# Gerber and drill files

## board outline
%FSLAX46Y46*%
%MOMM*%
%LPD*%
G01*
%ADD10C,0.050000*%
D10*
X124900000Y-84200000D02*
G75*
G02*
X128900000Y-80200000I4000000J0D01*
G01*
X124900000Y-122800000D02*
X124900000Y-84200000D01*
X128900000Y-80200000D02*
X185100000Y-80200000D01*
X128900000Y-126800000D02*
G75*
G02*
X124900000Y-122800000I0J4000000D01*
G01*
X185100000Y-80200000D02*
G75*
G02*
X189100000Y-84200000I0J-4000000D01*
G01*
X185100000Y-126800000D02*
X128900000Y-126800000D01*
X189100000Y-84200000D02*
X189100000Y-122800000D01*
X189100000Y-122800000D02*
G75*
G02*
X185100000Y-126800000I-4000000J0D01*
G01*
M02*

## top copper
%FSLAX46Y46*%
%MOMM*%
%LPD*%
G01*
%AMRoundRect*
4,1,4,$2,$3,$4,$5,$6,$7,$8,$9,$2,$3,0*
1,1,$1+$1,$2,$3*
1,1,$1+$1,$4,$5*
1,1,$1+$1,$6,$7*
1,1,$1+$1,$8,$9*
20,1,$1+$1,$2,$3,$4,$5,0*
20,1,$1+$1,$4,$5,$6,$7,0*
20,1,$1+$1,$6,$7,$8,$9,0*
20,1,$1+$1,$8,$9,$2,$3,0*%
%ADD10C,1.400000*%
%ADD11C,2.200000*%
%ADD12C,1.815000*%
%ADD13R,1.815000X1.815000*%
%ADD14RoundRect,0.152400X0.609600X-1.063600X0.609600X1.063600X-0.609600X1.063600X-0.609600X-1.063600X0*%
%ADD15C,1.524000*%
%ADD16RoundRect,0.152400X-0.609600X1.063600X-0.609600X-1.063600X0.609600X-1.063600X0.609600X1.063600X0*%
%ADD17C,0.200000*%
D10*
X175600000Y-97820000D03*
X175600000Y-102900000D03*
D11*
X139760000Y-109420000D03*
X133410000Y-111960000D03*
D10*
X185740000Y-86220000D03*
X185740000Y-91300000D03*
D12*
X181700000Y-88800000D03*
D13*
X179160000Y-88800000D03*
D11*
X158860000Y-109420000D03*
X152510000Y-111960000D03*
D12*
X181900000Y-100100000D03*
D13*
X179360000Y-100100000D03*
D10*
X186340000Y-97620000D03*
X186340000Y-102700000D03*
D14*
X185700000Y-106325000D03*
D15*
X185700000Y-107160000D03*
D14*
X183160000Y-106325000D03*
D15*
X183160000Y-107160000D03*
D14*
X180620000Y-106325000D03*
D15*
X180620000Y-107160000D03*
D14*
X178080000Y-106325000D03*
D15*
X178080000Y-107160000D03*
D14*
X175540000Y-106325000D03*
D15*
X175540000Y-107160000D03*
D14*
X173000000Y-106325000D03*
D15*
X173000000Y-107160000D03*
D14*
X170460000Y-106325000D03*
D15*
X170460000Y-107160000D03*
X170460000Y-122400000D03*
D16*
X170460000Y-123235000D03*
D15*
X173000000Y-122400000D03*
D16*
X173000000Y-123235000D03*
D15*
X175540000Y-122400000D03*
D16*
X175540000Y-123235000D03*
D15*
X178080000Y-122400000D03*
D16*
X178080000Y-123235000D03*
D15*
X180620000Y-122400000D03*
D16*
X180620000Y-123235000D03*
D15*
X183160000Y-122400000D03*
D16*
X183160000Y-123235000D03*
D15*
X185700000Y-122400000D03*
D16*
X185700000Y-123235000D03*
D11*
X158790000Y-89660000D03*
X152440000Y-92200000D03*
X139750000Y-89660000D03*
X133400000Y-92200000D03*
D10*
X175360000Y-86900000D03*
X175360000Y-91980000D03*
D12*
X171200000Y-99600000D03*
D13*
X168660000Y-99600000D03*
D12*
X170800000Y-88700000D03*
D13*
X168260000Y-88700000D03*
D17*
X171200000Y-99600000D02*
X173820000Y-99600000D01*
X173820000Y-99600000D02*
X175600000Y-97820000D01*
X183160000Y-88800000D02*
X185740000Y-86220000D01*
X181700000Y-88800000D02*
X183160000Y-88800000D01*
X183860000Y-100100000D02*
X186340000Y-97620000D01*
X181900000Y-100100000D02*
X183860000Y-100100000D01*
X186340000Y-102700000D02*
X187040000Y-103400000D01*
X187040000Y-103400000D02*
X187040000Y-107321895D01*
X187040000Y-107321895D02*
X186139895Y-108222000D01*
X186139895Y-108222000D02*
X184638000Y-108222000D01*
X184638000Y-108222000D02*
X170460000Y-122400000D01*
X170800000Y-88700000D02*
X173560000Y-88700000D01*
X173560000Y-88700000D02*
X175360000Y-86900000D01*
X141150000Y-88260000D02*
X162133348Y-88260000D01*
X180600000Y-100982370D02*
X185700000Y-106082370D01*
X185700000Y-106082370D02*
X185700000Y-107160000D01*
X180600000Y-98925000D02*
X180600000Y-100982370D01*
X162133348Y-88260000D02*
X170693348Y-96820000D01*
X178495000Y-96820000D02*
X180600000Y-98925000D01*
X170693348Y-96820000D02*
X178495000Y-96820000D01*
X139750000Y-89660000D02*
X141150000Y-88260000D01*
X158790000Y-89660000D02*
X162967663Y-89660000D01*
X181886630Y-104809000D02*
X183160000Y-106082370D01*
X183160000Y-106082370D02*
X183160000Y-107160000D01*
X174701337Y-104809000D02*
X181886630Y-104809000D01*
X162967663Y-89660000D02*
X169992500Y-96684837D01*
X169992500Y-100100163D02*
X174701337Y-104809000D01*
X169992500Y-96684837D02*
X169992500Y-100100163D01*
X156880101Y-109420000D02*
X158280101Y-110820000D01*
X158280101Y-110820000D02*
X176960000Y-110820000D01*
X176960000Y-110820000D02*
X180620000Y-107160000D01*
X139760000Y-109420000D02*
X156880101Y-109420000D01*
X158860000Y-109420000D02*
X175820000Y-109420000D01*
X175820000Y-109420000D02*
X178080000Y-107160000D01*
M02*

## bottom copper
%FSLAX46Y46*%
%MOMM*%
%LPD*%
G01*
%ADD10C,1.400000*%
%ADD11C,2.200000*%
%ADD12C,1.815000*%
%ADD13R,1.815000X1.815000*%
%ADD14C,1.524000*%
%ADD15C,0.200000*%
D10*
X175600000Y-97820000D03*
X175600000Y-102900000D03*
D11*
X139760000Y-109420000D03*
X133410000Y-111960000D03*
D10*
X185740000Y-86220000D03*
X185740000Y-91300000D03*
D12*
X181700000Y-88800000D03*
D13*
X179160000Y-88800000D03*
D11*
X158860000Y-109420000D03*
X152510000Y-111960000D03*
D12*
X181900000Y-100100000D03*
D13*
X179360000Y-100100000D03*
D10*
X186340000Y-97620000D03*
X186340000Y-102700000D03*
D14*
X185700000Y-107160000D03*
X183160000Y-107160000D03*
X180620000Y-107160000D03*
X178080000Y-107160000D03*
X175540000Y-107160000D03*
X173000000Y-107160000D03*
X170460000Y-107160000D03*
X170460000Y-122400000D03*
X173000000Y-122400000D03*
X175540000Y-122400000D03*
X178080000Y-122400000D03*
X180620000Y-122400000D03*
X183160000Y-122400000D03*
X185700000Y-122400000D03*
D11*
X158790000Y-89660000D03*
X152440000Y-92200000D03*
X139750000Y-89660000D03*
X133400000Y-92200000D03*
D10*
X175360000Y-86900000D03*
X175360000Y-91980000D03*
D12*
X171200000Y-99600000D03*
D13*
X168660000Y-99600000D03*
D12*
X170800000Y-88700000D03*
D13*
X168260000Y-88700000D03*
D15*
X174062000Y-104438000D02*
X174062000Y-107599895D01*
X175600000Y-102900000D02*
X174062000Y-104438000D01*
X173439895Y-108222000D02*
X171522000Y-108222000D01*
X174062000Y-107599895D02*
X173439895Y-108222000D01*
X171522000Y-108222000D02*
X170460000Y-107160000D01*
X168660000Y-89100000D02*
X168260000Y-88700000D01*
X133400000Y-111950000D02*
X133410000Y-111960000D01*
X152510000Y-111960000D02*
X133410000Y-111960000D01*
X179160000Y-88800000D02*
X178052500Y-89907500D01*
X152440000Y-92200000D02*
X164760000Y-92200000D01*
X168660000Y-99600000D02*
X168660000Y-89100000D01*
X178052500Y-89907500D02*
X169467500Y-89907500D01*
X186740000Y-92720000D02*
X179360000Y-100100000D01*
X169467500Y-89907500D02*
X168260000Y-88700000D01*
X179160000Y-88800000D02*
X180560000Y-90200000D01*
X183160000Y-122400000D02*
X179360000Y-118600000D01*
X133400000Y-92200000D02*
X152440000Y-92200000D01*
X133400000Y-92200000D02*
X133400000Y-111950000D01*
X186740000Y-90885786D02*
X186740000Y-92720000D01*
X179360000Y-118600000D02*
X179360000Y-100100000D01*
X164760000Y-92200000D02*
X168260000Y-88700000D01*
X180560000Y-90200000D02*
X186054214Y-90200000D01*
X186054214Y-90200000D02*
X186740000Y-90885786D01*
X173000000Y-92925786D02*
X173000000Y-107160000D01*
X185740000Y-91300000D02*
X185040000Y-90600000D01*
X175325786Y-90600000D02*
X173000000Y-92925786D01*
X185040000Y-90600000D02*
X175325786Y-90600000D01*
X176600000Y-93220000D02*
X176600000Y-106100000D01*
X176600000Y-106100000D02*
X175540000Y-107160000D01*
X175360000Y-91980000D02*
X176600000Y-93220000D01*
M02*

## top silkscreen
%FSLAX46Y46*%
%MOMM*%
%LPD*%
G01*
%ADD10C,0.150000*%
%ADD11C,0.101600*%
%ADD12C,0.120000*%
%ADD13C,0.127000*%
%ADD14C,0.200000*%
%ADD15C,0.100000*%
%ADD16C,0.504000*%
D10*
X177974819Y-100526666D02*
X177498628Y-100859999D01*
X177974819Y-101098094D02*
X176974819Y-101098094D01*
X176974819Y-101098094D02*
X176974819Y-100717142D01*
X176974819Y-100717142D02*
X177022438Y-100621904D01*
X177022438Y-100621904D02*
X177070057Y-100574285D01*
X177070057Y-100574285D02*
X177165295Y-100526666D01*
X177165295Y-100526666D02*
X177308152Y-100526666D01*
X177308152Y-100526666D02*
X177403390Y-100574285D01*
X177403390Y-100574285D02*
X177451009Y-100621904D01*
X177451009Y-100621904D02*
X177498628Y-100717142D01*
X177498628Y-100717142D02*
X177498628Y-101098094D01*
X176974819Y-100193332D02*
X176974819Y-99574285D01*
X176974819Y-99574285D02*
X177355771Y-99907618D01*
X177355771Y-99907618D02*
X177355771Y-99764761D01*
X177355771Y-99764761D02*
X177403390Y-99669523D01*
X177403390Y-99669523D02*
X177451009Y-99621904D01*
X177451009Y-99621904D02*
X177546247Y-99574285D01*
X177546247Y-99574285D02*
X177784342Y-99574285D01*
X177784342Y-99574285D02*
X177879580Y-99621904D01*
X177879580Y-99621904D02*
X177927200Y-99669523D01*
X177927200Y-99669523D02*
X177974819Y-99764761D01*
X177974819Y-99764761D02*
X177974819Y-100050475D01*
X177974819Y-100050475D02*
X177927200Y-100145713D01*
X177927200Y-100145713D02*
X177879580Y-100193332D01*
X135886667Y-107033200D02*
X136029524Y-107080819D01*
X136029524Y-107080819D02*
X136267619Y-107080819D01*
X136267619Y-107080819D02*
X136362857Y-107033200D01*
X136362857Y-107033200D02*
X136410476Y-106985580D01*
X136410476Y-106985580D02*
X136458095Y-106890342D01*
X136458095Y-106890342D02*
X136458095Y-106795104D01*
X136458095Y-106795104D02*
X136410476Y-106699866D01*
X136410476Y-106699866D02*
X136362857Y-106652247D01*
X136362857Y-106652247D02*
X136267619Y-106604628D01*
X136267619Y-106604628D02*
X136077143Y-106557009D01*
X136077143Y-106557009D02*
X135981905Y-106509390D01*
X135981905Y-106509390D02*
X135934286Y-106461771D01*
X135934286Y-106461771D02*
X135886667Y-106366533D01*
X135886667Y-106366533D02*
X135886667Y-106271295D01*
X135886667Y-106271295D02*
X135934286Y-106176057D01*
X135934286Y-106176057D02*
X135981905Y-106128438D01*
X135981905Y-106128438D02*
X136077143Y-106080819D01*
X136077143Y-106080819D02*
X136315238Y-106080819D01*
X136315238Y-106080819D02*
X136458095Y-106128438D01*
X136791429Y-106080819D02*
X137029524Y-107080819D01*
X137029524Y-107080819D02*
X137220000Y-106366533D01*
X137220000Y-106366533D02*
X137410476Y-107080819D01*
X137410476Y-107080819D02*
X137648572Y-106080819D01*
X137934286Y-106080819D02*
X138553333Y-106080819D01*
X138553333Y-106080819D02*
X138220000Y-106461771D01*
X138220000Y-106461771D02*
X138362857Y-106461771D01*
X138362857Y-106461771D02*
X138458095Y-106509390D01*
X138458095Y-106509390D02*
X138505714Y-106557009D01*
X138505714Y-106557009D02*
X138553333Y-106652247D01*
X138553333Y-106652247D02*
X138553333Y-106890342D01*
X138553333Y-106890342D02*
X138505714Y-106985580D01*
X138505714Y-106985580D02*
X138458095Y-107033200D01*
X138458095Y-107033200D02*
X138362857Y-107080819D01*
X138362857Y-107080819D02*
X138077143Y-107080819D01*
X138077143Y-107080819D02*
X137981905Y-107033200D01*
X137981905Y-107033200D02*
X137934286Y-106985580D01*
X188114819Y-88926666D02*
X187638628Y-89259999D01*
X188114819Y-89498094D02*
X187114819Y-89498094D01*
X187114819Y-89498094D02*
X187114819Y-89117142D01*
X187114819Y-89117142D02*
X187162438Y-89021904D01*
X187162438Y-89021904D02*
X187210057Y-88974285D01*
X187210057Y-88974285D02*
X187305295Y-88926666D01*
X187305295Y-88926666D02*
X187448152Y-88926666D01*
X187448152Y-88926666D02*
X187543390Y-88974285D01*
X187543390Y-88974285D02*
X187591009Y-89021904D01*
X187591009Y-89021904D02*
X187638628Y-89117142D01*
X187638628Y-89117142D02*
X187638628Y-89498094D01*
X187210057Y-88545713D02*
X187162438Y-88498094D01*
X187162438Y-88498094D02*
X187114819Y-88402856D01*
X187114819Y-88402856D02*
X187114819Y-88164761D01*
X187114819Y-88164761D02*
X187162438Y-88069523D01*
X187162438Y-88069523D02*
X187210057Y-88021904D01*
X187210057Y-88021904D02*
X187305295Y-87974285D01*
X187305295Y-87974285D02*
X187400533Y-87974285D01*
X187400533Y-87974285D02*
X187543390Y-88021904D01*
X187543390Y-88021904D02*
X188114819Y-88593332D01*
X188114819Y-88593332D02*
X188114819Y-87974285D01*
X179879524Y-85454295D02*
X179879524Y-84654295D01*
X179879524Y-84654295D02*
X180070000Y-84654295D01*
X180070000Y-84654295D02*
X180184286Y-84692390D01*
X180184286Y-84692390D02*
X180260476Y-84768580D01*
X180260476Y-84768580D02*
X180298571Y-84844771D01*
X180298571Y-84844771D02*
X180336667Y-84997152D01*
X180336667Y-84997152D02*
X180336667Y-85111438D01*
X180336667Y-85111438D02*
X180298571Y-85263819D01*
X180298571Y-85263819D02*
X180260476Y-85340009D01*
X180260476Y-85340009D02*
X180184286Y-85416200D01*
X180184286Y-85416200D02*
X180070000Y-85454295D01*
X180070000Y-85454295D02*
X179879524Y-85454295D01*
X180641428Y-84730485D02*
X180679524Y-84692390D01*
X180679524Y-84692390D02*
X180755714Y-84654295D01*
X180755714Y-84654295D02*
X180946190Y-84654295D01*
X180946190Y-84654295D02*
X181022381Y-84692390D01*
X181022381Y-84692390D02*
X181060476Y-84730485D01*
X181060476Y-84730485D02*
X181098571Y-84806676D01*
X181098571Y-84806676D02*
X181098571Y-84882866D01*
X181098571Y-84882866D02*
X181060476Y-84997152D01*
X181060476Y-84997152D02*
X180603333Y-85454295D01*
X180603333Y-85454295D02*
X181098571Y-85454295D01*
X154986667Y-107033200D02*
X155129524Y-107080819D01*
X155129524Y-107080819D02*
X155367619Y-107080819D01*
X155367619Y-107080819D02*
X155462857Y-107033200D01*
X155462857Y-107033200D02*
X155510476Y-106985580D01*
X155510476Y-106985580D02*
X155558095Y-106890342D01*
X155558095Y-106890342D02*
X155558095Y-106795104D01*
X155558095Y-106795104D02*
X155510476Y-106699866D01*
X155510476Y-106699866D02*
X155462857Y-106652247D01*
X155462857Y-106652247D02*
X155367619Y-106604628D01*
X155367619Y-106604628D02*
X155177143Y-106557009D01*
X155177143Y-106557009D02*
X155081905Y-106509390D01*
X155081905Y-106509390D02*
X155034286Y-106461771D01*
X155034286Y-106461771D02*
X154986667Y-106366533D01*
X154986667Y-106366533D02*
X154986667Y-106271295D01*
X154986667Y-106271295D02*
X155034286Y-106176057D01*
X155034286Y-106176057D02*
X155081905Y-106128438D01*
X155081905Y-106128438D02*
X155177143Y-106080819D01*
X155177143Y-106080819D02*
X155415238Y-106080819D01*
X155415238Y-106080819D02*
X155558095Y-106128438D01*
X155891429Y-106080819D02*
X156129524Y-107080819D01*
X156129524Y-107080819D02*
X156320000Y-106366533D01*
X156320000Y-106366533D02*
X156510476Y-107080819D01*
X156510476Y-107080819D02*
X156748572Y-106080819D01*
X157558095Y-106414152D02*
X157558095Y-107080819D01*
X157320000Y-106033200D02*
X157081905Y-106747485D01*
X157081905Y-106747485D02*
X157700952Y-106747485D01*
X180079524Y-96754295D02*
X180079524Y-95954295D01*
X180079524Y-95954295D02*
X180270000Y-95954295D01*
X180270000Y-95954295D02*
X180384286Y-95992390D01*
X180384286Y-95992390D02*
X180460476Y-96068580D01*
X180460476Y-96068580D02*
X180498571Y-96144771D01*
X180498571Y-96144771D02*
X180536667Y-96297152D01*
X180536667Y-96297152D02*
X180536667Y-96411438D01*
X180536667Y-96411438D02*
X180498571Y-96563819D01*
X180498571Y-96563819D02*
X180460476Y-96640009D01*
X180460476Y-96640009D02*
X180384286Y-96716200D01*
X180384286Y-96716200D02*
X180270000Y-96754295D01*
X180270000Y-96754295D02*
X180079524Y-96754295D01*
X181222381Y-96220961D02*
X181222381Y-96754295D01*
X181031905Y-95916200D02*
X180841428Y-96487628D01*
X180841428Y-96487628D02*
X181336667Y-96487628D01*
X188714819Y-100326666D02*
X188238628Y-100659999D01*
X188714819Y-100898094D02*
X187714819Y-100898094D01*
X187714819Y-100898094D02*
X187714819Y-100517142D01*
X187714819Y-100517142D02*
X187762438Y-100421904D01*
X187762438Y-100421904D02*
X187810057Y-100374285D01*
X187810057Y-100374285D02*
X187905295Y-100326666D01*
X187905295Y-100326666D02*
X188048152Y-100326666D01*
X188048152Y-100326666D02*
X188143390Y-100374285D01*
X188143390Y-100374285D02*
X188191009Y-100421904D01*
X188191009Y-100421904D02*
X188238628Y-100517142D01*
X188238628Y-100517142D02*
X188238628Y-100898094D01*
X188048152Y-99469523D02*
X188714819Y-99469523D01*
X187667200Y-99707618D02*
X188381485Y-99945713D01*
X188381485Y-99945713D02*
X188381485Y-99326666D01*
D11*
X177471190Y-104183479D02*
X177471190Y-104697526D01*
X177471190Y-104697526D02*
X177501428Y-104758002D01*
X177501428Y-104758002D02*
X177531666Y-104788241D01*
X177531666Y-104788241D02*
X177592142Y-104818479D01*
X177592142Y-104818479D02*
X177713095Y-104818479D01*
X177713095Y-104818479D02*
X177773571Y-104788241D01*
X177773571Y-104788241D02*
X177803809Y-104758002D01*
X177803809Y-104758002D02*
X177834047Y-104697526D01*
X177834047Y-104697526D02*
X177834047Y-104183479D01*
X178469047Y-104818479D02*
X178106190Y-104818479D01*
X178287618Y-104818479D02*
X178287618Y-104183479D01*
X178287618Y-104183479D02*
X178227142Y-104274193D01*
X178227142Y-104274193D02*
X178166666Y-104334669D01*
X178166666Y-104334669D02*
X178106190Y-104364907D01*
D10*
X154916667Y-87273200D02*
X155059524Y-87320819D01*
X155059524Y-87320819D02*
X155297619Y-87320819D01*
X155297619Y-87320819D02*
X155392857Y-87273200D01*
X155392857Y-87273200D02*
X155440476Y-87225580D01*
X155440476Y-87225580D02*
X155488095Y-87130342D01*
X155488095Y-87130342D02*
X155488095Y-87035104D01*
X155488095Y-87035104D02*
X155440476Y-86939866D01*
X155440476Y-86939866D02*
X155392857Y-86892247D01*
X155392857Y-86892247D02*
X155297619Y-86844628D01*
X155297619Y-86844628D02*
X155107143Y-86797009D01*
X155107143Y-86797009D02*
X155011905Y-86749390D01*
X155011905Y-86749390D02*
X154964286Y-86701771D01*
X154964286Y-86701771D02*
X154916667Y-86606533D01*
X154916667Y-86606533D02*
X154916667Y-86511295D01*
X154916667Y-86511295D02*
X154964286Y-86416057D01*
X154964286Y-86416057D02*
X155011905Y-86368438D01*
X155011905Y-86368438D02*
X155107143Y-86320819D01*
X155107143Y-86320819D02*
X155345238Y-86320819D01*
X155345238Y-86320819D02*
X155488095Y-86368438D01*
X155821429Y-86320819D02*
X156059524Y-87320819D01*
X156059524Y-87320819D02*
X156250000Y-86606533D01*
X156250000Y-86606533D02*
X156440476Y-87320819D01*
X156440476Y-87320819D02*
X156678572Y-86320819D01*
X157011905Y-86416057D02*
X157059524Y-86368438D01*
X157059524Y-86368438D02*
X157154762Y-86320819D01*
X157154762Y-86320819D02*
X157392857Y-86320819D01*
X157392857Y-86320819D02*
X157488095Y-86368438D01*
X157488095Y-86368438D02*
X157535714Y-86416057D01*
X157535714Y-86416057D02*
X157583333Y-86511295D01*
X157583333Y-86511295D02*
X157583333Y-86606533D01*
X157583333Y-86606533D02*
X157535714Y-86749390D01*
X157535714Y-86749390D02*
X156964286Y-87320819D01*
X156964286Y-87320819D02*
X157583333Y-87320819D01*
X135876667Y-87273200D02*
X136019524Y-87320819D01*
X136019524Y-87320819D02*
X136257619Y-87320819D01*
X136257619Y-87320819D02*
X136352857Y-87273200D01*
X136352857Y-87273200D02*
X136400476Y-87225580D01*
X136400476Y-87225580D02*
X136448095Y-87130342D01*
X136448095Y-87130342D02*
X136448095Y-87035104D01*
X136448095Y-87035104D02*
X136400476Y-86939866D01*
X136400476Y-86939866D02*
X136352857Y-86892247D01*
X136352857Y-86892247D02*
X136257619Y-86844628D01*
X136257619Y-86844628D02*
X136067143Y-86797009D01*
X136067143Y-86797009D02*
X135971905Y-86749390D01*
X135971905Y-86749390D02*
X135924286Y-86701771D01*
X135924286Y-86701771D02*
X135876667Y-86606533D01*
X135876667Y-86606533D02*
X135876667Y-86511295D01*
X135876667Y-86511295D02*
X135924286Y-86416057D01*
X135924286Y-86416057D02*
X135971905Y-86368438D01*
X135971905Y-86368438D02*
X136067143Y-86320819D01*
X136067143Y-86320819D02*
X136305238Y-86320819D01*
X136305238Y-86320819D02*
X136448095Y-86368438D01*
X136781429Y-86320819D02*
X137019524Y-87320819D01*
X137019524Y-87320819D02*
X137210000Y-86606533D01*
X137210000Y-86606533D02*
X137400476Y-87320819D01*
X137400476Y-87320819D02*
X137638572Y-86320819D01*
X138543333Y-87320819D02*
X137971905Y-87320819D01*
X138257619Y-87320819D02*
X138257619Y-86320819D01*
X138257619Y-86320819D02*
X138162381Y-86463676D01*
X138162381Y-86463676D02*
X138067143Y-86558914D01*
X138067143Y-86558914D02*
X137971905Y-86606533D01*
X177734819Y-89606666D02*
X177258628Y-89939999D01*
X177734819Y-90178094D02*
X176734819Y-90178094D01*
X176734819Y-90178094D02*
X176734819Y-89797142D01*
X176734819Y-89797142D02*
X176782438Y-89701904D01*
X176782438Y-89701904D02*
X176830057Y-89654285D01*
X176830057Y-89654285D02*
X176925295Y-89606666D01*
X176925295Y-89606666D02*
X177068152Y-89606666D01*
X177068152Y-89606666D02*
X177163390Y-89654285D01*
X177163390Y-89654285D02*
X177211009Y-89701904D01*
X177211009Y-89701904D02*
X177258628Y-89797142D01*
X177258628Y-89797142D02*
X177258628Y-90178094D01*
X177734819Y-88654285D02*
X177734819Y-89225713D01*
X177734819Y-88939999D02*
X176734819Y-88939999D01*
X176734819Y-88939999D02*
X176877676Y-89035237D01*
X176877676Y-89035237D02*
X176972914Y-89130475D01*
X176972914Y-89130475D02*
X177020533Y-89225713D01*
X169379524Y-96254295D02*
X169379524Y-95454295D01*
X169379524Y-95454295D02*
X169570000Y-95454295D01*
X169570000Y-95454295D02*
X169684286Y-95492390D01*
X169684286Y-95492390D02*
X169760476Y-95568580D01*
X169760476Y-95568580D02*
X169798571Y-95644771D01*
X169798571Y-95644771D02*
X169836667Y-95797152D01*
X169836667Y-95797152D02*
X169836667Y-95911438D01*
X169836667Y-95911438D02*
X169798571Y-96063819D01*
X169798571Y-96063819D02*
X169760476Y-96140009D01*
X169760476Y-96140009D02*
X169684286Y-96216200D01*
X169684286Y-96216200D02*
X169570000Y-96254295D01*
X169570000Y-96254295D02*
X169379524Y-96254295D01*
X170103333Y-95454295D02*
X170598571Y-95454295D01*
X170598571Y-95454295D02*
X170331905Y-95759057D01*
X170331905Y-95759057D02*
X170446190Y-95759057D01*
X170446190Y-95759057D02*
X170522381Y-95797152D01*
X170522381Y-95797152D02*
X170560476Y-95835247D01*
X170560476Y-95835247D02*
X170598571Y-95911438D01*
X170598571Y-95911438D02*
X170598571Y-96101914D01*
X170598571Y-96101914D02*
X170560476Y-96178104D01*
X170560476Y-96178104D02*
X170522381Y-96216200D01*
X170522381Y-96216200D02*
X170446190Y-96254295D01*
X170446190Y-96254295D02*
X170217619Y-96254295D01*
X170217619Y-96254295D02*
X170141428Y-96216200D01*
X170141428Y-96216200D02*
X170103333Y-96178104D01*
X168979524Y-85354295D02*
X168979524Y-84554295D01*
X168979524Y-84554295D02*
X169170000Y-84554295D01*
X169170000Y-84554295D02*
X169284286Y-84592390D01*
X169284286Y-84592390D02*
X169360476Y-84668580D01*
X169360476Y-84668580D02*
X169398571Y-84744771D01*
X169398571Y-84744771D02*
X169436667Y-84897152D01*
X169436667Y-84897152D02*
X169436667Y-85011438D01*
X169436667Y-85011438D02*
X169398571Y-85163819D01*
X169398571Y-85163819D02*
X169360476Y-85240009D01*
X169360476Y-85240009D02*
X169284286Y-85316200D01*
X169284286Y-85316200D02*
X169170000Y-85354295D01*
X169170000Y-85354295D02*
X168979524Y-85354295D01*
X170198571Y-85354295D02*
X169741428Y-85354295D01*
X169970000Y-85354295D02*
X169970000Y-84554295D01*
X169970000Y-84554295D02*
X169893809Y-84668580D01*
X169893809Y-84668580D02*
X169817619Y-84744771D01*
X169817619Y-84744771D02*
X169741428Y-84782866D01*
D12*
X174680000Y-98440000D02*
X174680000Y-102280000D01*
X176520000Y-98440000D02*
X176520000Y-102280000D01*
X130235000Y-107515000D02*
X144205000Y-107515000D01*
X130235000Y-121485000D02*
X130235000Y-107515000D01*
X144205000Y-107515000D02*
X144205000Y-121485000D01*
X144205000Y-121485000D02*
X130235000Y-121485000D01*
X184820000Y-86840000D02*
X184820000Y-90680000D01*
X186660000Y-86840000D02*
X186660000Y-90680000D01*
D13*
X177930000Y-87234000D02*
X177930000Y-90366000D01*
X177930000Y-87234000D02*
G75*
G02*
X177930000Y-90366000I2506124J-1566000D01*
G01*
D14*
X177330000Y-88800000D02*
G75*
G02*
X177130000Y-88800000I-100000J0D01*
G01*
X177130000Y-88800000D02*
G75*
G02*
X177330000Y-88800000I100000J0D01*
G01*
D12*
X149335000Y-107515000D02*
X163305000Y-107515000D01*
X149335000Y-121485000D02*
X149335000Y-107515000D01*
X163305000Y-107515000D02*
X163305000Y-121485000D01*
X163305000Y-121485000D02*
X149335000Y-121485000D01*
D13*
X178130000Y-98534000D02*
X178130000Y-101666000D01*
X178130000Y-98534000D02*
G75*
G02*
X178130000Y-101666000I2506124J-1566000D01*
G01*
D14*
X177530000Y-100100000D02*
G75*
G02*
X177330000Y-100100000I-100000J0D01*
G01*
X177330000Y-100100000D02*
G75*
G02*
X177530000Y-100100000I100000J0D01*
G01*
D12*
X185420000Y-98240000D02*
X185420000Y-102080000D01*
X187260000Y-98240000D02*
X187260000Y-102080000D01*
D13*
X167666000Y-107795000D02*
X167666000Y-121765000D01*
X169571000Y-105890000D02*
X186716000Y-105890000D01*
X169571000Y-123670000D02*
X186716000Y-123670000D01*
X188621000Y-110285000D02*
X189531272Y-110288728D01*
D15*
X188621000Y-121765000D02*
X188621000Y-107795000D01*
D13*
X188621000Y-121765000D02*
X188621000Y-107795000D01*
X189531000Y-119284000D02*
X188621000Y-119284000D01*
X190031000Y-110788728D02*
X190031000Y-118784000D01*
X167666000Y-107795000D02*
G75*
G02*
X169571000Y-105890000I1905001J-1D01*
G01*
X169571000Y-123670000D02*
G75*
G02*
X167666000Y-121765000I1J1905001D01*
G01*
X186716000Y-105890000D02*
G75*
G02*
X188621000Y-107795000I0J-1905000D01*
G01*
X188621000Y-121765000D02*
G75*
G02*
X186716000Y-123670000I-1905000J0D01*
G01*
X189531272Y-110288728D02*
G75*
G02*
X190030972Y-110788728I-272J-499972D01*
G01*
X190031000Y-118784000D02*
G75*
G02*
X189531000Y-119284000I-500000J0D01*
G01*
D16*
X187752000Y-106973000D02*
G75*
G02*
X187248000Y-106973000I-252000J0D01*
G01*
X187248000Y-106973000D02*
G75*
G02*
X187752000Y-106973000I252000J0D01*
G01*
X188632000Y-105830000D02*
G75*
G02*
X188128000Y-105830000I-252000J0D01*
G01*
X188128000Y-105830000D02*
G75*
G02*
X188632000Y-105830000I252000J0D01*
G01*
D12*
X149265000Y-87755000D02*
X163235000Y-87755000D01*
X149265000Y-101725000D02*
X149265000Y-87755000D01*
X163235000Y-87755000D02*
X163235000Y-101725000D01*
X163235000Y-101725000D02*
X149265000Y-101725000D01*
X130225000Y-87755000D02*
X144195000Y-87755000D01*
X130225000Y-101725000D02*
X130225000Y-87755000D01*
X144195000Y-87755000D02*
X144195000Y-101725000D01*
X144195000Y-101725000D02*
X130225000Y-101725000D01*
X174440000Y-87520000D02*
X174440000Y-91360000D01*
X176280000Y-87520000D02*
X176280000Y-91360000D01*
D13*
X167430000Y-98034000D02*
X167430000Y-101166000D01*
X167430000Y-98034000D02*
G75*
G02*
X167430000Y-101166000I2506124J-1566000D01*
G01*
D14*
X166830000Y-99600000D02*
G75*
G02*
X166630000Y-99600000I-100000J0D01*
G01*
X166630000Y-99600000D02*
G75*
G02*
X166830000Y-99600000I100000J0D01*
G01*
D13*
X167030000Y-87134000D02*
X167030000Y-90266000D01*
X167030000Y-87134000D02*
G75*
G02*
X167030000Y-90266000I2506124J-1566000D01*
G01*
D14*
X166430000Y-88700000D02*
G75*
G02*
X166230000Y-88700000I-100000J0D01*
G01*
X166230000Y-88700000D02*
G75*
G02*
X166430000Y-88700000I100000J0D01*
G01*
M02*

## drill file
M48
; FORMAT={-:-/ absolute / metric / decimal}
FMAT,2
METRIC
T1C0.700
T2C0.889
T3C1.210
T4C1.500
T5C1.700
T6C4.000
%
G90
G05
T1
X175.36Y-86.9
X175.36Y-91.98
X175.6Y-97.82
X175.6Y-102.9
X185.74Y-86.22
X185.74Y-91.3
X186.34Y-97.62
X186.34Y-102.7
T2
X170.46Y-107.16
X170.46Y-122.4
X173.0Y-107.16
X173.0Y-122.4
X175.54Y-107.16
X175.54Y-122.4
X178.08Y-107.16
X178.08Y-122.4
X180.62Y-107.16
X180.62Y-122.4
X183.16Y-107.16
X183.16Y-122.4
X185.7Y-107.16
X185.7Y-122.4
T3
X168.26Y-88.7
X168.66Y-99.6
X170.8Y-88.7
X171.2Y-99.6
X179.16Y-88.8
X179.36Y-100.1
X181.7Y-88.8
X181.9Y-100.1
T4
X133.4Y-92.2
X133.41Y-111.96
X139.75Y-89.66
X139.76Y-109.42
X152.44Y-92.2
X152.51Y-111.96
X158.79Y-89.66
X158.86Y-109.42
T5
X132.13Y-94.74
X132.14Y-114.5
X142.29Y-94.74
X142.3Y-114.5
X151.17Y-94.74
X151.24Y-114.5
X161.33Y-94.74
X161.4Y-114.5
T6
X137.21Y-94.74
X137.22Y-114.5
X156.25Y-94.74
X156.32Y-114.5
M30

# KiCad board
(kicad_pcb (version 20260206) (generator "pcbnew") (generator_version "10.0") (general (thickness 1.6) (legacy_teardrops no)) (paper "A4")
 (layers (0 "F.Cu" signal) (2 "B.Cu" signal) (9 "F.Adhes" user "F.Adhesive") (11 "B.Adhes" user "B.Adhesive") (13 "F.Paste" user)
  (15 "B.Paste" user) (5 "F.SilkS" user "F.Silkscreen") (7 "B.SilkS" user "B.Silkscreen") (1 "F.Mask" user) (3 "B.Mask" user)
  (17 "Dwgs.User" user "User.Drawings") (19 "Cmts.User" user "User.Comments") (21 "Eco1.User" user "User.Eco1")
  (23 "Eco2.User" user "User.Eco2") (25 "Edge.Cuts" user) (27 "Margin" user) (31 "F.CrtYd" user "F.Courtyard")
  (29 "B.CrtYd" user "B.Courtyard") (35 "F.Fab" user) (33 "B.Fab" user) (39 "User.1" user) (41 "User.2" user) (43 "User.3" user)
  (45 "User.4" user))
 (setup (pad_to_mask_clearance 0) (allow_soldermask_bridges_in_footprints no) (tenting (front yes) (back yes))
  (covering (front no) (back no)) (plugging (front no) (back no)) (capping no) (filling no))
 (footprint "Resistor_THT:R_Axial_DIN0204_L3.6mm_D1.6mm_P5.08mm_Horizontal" (layer "F.Cu") (at 175.6 97.82 -90)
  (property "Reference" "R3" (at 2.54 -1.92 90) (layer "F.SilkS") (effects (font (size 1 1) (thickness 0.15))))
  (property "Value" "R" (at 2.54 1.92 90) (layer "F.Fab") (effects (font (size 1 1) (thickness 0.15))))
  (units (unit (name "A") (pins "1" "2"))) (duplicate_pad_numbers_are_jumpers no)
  (fp_line (start 0.62 0.92) (end 4.46 0.92) (stroke (width 0.12) (type solid)) (layer "F.SilkS"))
  (fp_line (start 0.62 -0.92) (end 4.46 -0.92) (stroke (width 0.12) (type solid)) (layer "F.SilkS"))
  (pad "1" thru_hole circle (at 0 0 270) (size 1.4 1.4) (drill 0.7) (layers "*.Cu" "*.Mask") (remove_unused_layers no) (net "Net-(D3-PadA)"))
  (pad "2" thru_hole circle (at 5.08 0 270) (size 1.4 1.4) (drill 0.7) (layers "*.Cu" "*.Mask") (remove_unused_layers no) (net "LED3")))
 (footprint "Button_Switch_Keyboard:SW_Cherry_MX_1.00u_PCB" (layer "F.Cu") (at 139.76 109.42)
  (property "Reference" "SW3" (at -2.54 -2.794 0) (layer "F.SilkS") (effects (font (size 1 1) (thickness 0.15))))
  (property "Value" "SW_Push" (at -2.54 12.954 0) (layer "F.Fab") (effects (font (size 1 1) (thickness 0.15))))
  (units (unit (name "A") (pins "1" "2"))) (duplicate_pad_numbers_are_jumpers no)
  (fp_line (start -9.525 -1.905) (end 4.445 -1.905) (stroke (width 0.12) (type solid)) (layer "F.SilkS"))
  (fp_line (start -9.525 12.065) (end -9.525 -1.905) (stroke (width 0.12) (type solid)) (layer "F.SilkS"))
  (fp_line (start 4.445 -1.905) (end 4.445 12.065) (stroke (width 0.12) (type solid)) (layer "F.SilkS"))
  (fp_line (start 4.445 12.065) (end -9.525 12.065) (stroke (width 0.12) (type solid)) (layer "F.SilkS"))
  (pad "" np_thru_hole circle (at -7.62 5.08) (size 1.7 1.7) (drill 1.7) (layers "*.Cu" "*.Mask"))
  (pad "" np_thru_hole circle (at -2.54 5.08) (size 4 4) (drill 4) (layers "*.Cu" "*.Mask"))
  (pad "" np_thru_hole circle (at 2.54 5.08) (size 1.7 1.7) (drill 1.7) (layers "*.Cu" "*.Mask"))
  (pad "1" thru_hole circle (at 0 0) (size 2.2 2.2) (drill 1.5) (layers "*.Cu" "*.Mask") (remove_unused_layers no) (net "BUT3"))
  (pad "2" thru_hole circle (at -6.35 2.54) (size 2.2 2.2) (drill 1.5) (layers "*.Cu" "*.Mask") (remove_unused_layers no) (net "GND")))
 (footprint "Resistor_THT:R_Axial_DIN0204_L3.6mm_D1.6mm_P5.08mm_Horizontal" (layer "F.Cu") (at 185.74 86.22 -90)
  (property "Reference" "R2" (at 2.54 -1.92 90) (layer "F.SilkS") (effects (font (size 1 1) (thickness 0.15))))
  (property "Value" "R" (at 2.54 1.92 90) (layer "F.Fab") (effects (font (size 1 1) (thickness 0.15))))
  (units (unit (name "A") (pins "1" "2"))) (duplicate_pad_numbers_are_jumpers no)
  (fp_line (start 0.62 0.92) (end 4.46 0.92) (stroke (width 0.12) (type solid)) (layer "F.SilkS"))
  (fp_line (start 0.62 -0.92) (end 4.46 -0.92) (stroke (width 0.12) (type solid)) (layer "F.SilkS"))
  (pad "1" thru_hole circle (at 0 0 270) (size 1.4 1.4) (drill 0.7) (layers "*.Cu" "*.Mask") (remove_unused_layers no) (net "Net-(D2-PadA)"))
  (pad "2" thru_hole circle (at 5.08 0 270) (size 1.4 1.4) (drill 0.7) (layers "*.Cu" "*.Mask") (remove_unused_layers no) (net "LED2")))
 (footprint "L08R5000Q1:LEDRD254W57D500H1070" (layer "F.Cu") (at 180.43 88.8)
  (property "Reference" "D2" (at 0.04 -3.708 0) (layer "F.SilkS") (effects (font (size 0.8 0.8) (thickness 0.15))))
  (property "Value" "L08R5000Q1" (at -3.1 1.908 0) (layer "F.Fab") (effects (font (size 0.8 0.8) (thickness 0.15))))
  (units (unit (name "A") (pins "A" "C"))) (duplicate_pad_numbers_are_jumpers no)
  (fp_line (start -2.5 -1.566) (end -2.5 1.566) (stroke (width 0.127) (type solid)) (layer "F.SilkS"))
  (fp_arc (start -2.5 -1.566) (mid 2.961291 0) (end -2.5 1.566) (stroke (width 0.127) (type solid)) (layer "F.SilkS"))
  (fp_circle (center -3.2 0) (end -3.1 0) (stroke (width 0.2) (type solid)) (fill no) (layer "F.SilkS"))
  (pad "A" thru_hole circle (at 1.27 0) (size 1.815 1.815) (drill 1.21) (layers "*.Cu" "*.Mask") (remove_unused_layers no)
   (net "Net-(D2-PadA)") (solder_mask_margin 0.102))
  (pad "C" thru_hole rect (at -1.27 0) (size 1.815 1.815) (drill 1.21) (layers "*.Cu" "*.Mask") (remove_unused_layers no) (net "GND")
   (solder_mask_margin 0.102)))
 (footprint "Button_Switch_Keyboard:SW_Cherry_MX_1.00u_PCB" (layer "F.Cu") (at 158.86 109.42)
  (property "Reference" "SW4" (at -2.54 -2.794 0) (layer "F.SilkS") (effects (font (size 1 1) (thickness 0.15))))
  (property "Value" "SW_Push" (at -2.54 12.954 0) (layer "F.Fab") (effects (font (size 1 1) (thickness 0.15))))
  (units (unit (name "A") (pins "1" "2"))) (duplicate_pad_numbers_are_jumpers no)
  (fp_line (start -9.525 -1.905) (end 4.445 -1.905) (stroke (width 0.12) (type solid)) (layer "F.SilkS"))
  (fp_line (start -9.525 12.065) (end -9.525 -1.905) (stroke (width 0.12) (type solid)) (layer "F.SilkS"))
  (fp_line (start 4.445 -1.905) (end 4.445 12.065) (stroke (width 0.12) (type solid)) (layer "F.SilkS"))
  (fp_line (start 4.445 12.065) (end -9.525 12.065) (stroke (width 0.12) (type solid)) (layer "F.SilkS"))
  (pad "" np_thru_hole circle (at -7.62 5.08) (size 1.7 1.7) (drill 1.7) (layers "*.Cu" "*.Mask"))
  (pad "" np_thru_hole circle (at -2.54 5.08) (size 4 4) (drill 4) (layers "*.Cu" "*.Mask"))
  (pad "" np_thru_hole circle (at 2.54 5.08) (size 1.7 1.7) (drill 1.7) (layers "*.Cu" "*.Mask"))
  (pad "1" thru_hole circle (at 0 0) (size 2.2 2.2) (drill 1.5) (layers "*.Cu" "*.Mask") (remove_unused_layers no) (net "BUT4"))
  (pad "2" thru_hole circle (at -6.35 2.54) (size 2.2 2.2) (drill 1.5) (layers "*.Cu" "*.Mask") (remove_unused_layers no) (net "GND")))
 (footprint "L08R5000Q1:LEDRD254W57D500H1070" (layer "F.Cu") (at 180.63 100.1)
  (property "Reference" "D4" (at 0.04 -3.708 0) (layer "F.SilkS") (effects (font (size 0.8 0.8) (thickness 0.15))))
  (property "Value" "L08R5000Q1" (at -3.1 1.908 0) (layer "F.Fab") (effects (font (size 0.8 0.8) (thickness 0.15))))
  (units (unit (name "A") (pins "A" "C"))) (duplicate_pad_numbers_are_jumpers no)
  (fp_line (start -2.5 -1.566) (end -2.5 1.566) (stroke (width 0.127) (type solid)) (layer "F.SilkS"))
  (fp_arc (start -2.5 -1.566) (mid 2.961291 0) (end -2.5 1.566) (stroke (width 0.127) (type solid)) (layer "F.SilkS"))
  (fp_circle (center -3.2 0) (end -3.1 0) (stroke (width 0.2) (type solid)) (fill no) (layer "F.SilkS"))
  (pad "A" thru_hole circle (at 1.27 0) (size 1.815 1.815) (drill 1.21) (layers "*.Cu" "*.Mask") (remove_unused_layers no)
   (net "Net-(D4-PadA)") (solder_mask_margin 0.102))
  (pad "C" thru_hole rect (at -1.27 0) (size 1.815 1.815) (drill 1.21) (layers "*.Cu" "*.Mask") (remove_unused_layers no) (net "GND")
   (solder_mask_margin 0.102)))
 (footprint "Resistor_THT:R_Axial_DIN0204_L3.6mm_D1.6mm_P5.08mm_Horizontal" (layer "F.Cu") (at 186.34 97.62 -90)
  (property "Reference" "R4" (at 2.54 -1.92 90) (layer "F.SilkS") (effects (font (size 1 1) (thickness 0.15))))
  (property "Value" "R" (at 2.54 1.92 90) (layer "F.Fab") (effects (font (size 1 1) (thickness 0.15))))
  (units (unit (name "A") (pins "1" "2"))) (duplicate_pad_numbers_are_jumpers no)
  (fp_line (start 0.62 0.92) (end 4.46 0.92) (stroke (width 0.12) (type solid)) (layer "F.SilkS"))
  (fp_line (start 0.62 -0.92) (end 4.46 -0.92) (stroke (width 0.12) (type solid)) (layer "F.SilkS"))
  (pad "1" thru_hole circle (at 0 0 270) (size 1.4 1.4) (drill 0.7) (layers "*.Cu" "*.Mask") (remove_unused_layers no) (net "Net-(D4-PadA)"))
  (pad "2" thru_hole circle (at 5.08 0 270) (size 1.4 1.4) (drill 0.7) (layers "*.Cu" "*.Mask") (remove_unused_layers no) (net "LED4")))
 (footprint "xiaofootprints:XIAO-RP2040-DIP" (layer "F.Cu") (at 178.08 114.78)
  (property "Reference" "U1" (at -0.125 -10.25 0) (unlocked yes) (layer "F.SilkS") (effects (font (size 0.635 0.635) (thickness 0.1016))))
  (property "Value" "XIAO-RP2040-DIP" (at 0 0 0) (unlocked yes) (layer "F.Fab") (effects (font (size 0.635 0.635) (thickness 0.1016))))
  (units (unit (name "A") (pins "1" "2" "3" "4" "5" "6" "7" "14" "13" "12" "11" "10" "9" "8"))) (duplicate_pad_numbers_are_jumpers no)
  (fp_line (start -10.414 -6.985) (end -10.414 6.985) (stroke (width 0.127) (type solid)) (layer "F.SilkS"))
  (fp_line (start -8.509 -8.89) (end 8.636 -8.89) (stroke (width 0.127) (type solid)) (layer "F.SilkS"))
  (fp_line (start -8.509 8.89) (end 8.636 8.89) (stroke (width 0.127) (type solid)) (layer "F.SilkS"))
  (fp_line (start 10.541 -4.495) (end 11.451272 -4.491272) (stroke (width 0.127) (type solid)) (layer "F.SilkS"))
  (fp_line (start 10.541 6.985) (end 10.541 -6.985) (stroke (width 0.1) (type solid)) (layer "F.SilkS"))
  (fp_line (start 10.541 6.985) (end 10.541 -6.985) (stroke (width 0.127) (type solid)) (layer "F.SilkS"))
  (fp_line (start 11.451 4.504) (end 10.541 4.504) (stroke (width 0.127) (type solid)) (layer "F.SilkS"))
  (fp_line (start 11.951 -3.991272) (end 11.951 4.004) (stroke (width 0.127) (type solid)) (layer "F.SilkS"))
  (fp_arc (start -10.414 -6.985) (mid -9.856038 -8.332038) (end -8.509 -8.89) (stroke (width 0.127) (type solid)) (layer "F.SilkS"))
  (fp_arc (start -8.509 8.89) (mid -9.856038 8.332038) (end -10.414 6.985) (stroke (width 0.127) (type solid)) (layer "F.SilkS"))
  (fp_arc (start 8.636 -8.89) (mid 9.983038 -8.332038) (end 10.541 -6.985) (stroke (width 0.127) (type solid)) (layer "F.SilkS"))
  (fp_arc (start 10.541 6.985) (mid 9.983038 8.332038) (end 8.636 8.89) (stroke (width 0.127) (type solid)) (layer "F.SilkS"))
  (fp_arc (start 11.451272 -4.491272) (mid 11.804644 -4.344724) (end 11.951 -3.991272) (stroke (width 0.127) (type default))
   (layer "F.SilkS"))
  (fp_arc (start 11.951 4.004) (mid 11.804553 4.357553) (end 11.451 4.504) (stroke (width 0.127) (type default)) (layer "F.SilkS"))
  (fp_circle (center 9.42 -7.807) (end 9.674 -7.807) (stroke (width 0.5) (type solid)) (fill yes) (layer "F.SilkS"))
  (fp_circle (center 10.3 -8.95) (end 10.554 -8.95) (stroke (width 0.5) (type solid)) (fill yes) (layer "F.SilkS"))
  (pad "1" smd roundrect (at 7.62 -8.455 90) (size 2.432 1.524) (layers "F.Cu" "F.Mask") (roundrect_rratio 0.1) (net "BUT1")
   (thermal_bridge_angle 45))
  (pad "1" thru_hole circle (at 7.62 -7.62 90) (size 1.524 1.524) (drill 0.889) (layers "*.Cu" "*.Mask") (remove_unused_layers no)
   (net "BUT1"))
  (pad "2" smd roundrect (at 5.08 -8.455 90) (size 2.432 1.524) (layers "F.Cu" "F.Mask") (roundrect_rratio 0.1) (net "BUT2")
   (thermal_bridge_angle 45))
  (pad "2" thru_hole circle (at 5.08 -7.62 90) (size 1.524 1.524) (drill 0.889) (layers "*.Cu" "*.Mask") (remove_unused_layers no)
   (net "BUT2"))
  (pad "3" smd roundrect (at 2.54 -8.455 90) (size 2.432 1.524) (layers "F.Cu" "F.Mask") (roundrect_rratio 0.1) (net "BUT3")
   (thermal_bridge_angle 45))
  (pad "3" thru_hole circle (at 2.54 -7.62 90) (size 1.524 1.524) (drill 0.889) (layers "*.Cu" "*.Mask") (remove_unused_layers no)
   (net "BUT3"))
  (pad "4" smd roundrect (at 0 -8.455 90) (size 2.432 1.524) (layers "F.Cu" "F.Mask") (roundrect_rratio 0.1) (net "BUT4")
   (thermal_bridge_angle 45))
  (pad "4" thru_hole circle (at 0 -7.62 90) (size 1.524 1.524) (drill 0.889) (layers "*.Cu" "*.Mask") (remove_unused_layers no) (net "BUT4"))
  (pad "5" smd roundrect (at -2.54 -8.455 90) (size 2.432 1.524) (layers "F.Cu" "F.Mask") (roundrect_rratio 0.1) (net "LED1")
   (thermal_bridge_angle 45))
  (pad "5" thru_hole circle (at -2.54 -7.62 90) (size 1.524 1.524) (drill 0.889) (layers "*.Cu" "*.Mask") (remove_unused_layers no)
   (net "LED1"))
  (pad "6" smd roundrect (at -5.08 -8.455 90) (size 2.432 1.524) (layers "F.Cu" "F.Mask") (roundrect_rratio 0.1) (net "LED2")
   (thermal_bridge_angle 45))
  (pad "6" thru_hole circle (at -5.08 -7.62 90) (size 1.524 1.524) (drill 0.889) (layers "*.Cu" "*.Mask") (remove_unused_layers no)
   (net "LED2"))
  (pad "7" smd roundrect (at -7.62 -8.455 90) (size 2.432 1.524) (layers "F.Cu" "F.Mask") (roundrect_rratio 0.1) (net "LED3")
   (thermal_bridge_angle 45))
  (pad "7" thru_hole circle (at -7.62 -7.62 90) (size 1.524 1.524) (drill 0.889) (layers "*.Cu" "*.Mask") (remove_unused_layers no)
   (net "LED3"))
  (pad "8" thru_hole circle (at -7.62 7.62 270) (size 1.524 1.524) (drill 0.889) (layers "*.Cu" "*.Mask") (remove_unused_layers no)
   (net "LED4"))
  (pad "8" smd roundrect (at -7.62 8.455 270) (size 2.432 1.524) (layers "F.Cu" "F.Mask") (roundrect_rratio 0.1) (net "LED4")
   (thermal_bridge_angle 45))
  (pad "9" thru_hole circle (at -5.08 7.62 270) (size 1.524 1.524) (drill 0.889) (layers "*.Cu" "*.Mask") (remove_unused_layers no)
   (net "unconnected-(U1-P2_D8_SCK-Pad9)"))
  (pad "9" smd roundrect (at -5.08 8.455 270) (size 2.432 1.524) (layers "F.Cu" "F.Mask") (roundrect_rratio 0.1)
   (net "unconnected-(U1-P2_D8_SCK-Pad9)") (thermal_bridge_angle 45))
  (pad "10" thru_hole circle (at -2.54 7.62 270) (size 1.524 1.524) (drill 0.889) (layers "*.Cu" "*.Mask") (remove_unused_layers no)
   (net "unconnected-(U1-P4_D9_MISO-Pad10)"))
  (pad "10" smd roundrect (at -2.54 8.455 270) (size 2.432 1.524) (layers "F.Cu" "F.Mask") (roundrect_rratio 0.1)
   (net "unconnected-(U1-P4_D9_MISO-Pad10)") (thermal_bridge_angle 45))
  (pad "11" thru_hole circle (at 0 7.62 270) (size 1.524 1.524) (drill 0.889) (layers "*.Cu" "*.Mask") (remove_unused_layers no)
   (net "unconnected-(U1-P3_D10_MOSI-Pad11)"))
  (pad "11" smd roundrect (at 0 8.455 270) (size 2.432 1.524) (layers "F.Cu" "F.Mask") (roundrect_rratio 0.1)
   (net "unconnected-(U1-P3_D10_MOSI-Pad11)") (thermal_bridge_angle 45))
  (pad "12" thru_hole circle (at 2.54 7.62 270) (size 1.524 1.524) (drill 0.889) (layers "*.Cu" "*.Mask") (remove_unused_layers no)
   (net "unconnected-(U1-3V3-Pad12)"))
  (pad "12" smd roundrect (at 2.54 8.455 270) (size 2.432 1.524) (layers "F.Cu" "F.Mask") (roundrect_rratio 0.1)
   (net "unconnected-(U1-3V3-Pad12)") (thermal_bridge_angle 45))
  (pad "13" thru_hole circle (at 5.08 7.62 270) (size 1.524 1.524) (drill 0.889) (layers "*.Cu" "*.Mask") (remove_unused_layers no)
   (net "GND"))
  (pad "13" smd roundrect (at 5.08 8.455 270) (size 2.432 1.524) (layers "F.Cu" "F.Mask") (roundrect_rratio 0.1) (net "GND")
   (thermal_bridge_angle 45))
  (pad "14" thru_hole circle (at 7.62 7.62 270) (size 1.524 1.524) (drill 0.889) (layers "*.Cu" "*.Mask") (remove_unused_layers no)
   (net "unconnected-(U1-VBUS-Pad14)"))
  (pad "14" smd roundrect (at 7.62 8.455 270) (size 2.432 1.524) (layers "F.Cu" "F.Mask") (roundrect_rratio 0.1)
   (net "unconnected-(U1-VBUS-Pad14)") (thermal_bridge_angle 45)))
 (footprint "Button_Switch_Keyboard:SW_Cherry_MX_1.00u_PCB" (layer "F.Cu") (at 158.79 89.66)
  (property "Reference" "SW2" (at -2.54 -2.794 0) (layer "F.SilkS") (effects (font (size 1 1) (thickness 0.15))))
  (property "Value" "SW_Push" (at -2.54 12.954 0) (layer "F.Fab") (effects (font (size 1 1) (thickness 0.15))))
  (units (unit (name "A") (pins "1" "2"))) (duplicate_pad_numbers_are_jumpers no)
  (fp_line (start -9.525 -1.905) (end 4.445 -1.905) (stroke (width 0.12) (type solid)) (layer "F.SilkS"))
  (fp_line (start -9.525 12.065) (end -9.525 -1.905) (stroke (width 0.12) (type solid)) (layer "F.SilkS"))
  (fp_line (start 4.445 -1.905) (end 4.445 12.065) (stroke (width 0.12) (type solid)) (layer "F.SilkS"))
  (fp_line (start 4.445 12.065) (end -9.525 12.065) (stroke (width 0.12) (type solid)) (layer "F.SilkS"))
  (pad "" np_thru_hole circle (at -7.62 5.08) (size 1.7 1.7) (drill 1.7) (layers "*.Cu" "*.Mask"))
  (pad "" np_thru_hole circle (at -2.54 5.08) (size 4 4) (drill 4) (layers "*.Cu" "*.Mask"))
  (pad "" np_thru_hole circle (at 2.54 5.08) (size 1.7 1.7) (drill 1.7) (layers "*.Cu" "*.Mask"))
  (pad "1" thru_hole circle (at 0 0) (size 2.2 2.2) (drill 1.5) (layers "*.Cu" "*.Mask") (remove_unused_layers no) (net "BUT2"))
  (pad "2" thru_hole circle (at -6.35 2.54) (size 2.2 2.2) (drill 1.5) (layers "*.Cu" "*.Mask") (remove_unused_layers no) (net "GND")))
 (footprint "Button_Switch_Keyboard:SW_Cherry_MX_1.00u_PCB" (layer "F.Cu") (at 139.75 89.66)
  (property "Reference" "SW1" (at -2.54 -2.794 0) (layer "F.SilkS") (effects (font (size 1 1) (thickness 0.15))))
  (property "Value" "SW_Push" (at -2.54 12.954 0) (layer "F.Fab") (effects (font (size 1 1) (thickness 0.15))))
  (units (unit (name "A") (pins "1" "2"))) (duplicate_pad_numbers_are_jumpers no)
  (fp_line (start -9.525 -1.905) (end 4.445 -1.905) (stroke (width 0.12) (type solid)) (layer "F.SilkS"))
  (fp_line (start -9.525 12.065) (end -9.525 -1.905) (stroke (width 0.12) (type solid)) (layer "F.SilkS"))
  (fp_line (start 4.445 -1.905) (end 4.445 12.065) (stroke (width 0.12) (type solid)) (layer "F.SilkS"))
  (fp_line (start 4.445 12.065) (end -9.525 12.065) (stroke (width 0.12) (type solid)) (layer "F.SilkS"))
  (pad "" np_thru_hole circle (at -7.62 5.08) (size 1.7 1.7) (drill 1.7) (layers "*.Cu" "*.Mask"))
  (pad "" np_thru_hole circle (at -2.54 5.08) (size 4 4) (drill 4) (layers "*.Cu" "*.Mask"))
  (pad "" np_thru_hole circle (at 2.54 5.08) (size 1.7 1.7) (drill 1.7) (layers "*.Cu" "*.Mask"))
  (pad "1" thru_hole circle (at 0 0) (size 2.2 2.2) (drill 1.5) (layers "*.Cu" "*.Mask") (remove_unused_layers no) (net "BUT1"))
  (pad "2" thru_hole circle (at -6.35 2.54) (size 2.2 2.2) (drill 1.5) (layers "*.Cu" "*.Mask") (remove_unused_layers no) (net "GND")))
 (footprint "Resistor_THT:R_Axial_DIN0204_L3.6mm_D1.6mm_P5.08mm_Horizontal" (layer "F.Cu") (at 175.36 86.9 -90)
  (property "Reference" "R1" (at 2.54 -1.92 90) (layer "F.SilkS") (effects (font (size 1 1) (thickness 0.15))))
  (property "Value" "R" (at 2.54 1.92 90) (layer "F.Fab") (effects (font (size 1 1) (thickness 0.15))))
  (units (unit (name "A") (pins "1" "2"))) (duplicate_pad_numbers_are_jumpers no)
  (fp_line (start 0.62 0.92) (end 4.46 0.92) (stroke (width 0.12) (type solid)) (layer "F.SilkS"))
  (fp_line (start 0.62 -0.92) (end 4.46 -0.92) (stroke (width 0.12) (type solid)) (layer "F.SilkS"))
  (pad "1" thru_hole circle (at 0 0 270) (size 1.4 1.4) (drill 0.7) (layers "*.Cu" "*.Mask") (remove_unused_layers no) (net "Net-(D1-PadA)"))
  (pad "2" thru_hole circle (at 5.08 0 270) (size 1.4 1.4) (drill 0.7) (layers "*.Cu" "*.Mask") (remove_unused_layers no) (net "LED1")))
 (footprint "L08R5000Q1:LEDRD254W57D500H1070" (layer "F.Cu") (at 169.93 99.6)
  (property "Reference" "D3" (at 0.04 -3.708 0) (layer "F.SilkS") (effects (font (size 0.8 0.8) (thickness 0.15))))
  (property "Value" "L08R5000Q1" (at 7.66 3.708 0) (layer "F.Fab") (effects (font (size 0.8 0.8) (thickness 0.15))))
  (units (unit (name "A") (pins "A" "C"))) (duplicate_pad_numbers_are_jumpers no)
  (fp_line (start -2.5 -1.566) (end -2.5 1.566) (stroke (width 0.127) (type solid)) (layer "F.SilkS"))
  (fp_arc (start -2.5 -1.566) (mid 2.961291 0) (end -2.5 1.566) (stroke (width 0.127) (type solid)) (layer "F.SilkS"))
  (fp_circle (center -3.2 0) (end -3.1 0) (stroke (width 0.2) (type solid)) (fill no) (layer "F.SilkS"))
  (pad "A" thru_hole circle (at 1.27 0) (size 1.815 1.815) (drill 1.21) (layers "*.Cu" "*.Mask") (remove_unused_layers no)
   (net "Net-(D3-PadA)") (solder_mask_margin 0.102))
  (pad "C" thru_hole rect (at -1.27 0) (size 1.815 1.815) (drill 1.21) (layers "*.Cu" "*.Mask") (remove_unused_layers no) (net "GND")
   (solder_mask_margin 0.102)))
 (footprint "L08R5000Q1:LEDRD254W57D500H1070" (layer "F.Cu") (at 169.53 88.7)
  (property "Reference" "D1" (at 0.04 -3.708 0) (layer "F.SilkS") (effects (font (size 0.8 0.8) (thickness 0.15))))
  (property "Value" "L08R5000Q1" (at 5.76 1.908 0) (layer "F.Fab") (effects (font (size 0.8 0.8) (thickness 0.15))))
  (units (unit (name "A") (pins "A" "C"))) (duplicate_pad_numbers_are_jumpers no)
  (fp_line (start -2.5 -1.566) (end -2.5 1.566) (stroke (width 0.127) (type solid)) (layer "F.SilkS"))
  (fp_arc (start -2.5 -1.566) (mid 2.961291 0) (end -2.5 1.566) (stroke (width 0.127) (type solid)) (layer "F.SilkS"))
  (fp_circle (center -3.2 0) (end -3.1 0) (stroke (width 0.2) (type solid)) (fill no) (layer "F.SilkS"))
  (pad "A" thru_hole circle (at 1.27 0) (size 1.815 1.815) (drill 1.21) (layers "*.Cu" "*.Mask") (remove_unused_layers no)
   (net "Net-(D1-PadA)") (solder_mask_margin 0.102))
  (pad "C" thru_hole rect (at -1.27 0) (size 1.815 1.815) (drill 1.21) (layers "*.Cu" "*.Mask") (remove_unused_layers no) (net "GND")
   (solder_mask_margin 0.102)))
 (gr_arc (start 124.9 84.2) (mid 126.071573 81.371573) (end 128.9 80.2) (stroke (width 0.05) (type default)) (layer "Edge.Cuts"))
 (gr_line (start 124.9 122.8) (end 124.9 84.2) (stroke (width 0.05) (type default)) (layer "Edge.Cuts"))
 (gr_line (start 128.9 80.2) (end 185.1 80.2) (stroke (width 0.05) (type default)) (layer "Edge.Cuts"))
 (gr_arc (start 128.9 126.8) (mid 126.071573 125.628427) (end 124.9 122.8) (stroke (width 0.05) (type default)) (layer "Edge.Cuts"))
 (gr_arc (start 185.1 80.2) (mid 187.928427 81.371573) (end 189.1 84.2) (stroke (width 0.05) (type default)) (layer "Edge.Cuts"))
 (gr_line (start 185.1 126.8) (end 128.9 126.8) (stroke (width 0.05) (type default)) (layer "Edge.Cuts"))
 (gr_line (start 189.1 84.2) (end 189.1 122.8) (stroke (width 0.05) (type default)) (layer "Edge.Cuts"))
 (gr_arc (start 189.1 122.8) (mid 187.928427 125.628427) (end 185.1 126.8) (stroke (width 0.05) (type default)) (layer "Edge.Cuts"))
 (segment (start 171.2 99.6) (end 173.82 99.6) (width 0.2) (layer "F.Cu") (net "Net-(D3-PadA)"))
 (segment (start 173.82 99.6) (end 175.6 97.82) (width 0.2) (layer "F.Cu") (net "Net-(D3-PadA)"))
 (segment (start 174.062 104.438) (end 174.062 107.599895) (width 0.2) (layer "B.Cu") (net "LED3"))
 (segment (start 175.6 102.9) (end 174.062 104.438) (width 0.2) (layer "B.Cu") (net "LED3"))
 (segment (start 173.439895 108.222) (end 171.522 108.222) (width 0.2) (layer "B.Cu") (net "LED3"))
 (segment (start 174.062 107.599895) (end 173.439895 108.222) (width 0.2) (layer "B.Cu") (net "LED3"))
 (segment (start 171.522 108.222) (end 170.46 107.16) (width 0.2) (layer "B.Cu") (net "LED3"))
 (segment (start 168.66 89.1) (end 168.26 88.7) (width 0.2) (layer "B.Cu") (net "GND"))
 (segment (start 133.4 111.95) (end 133.41 111.96) (width 0.2) (layer "B.Cu") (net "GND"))
 (segment (start 152.51 111.96) (end 133.41 111.96) (width 0.2) (layer "B.Cu") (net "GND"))
 (segment (start 179.16 88.8) (end 178.0525 89.9075) (width 0.2) (layer "B.Cu") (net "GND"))
 (segment (start 152.44 92.2) (end 164.76 92.2) (width 0.2) (layer "B.Cu") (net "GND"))
 (segment (start 168.66 99.6) (end 168.66 89.1) (width 0.2) (layer "B.Cu") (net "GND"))
 (segment (start 178.0525 89.9075) (end 169.4675 89.9075) (width 0.2) (layer "B.Cu") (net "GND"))
 (segment (start 186.74 92.72) (end 179.36 100.1) (width 0.2) (layer "B.Cu") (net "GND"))
 (segment (start 169.4675 89.9075) (end 168.26 88.7) (width 0.2) (layer "B.Cu") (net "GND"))
 (segment (start 179.16 88.8) (end 180.56 90.2) (width 0.2) (layer "B.Cu") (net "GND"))
 (segment (start 183.16 122.4) (end 179.36 118.6) (width 0.2) (layer "B.Cu") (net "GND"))
 (segment (start 133.4 92.2) (end 152.44 92.2) (width 0.2) (layer "B.Cu") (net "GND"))
 (segment (start 133.4 92.2) (end 133.4 111.95) (width 0.2) (layer "B.Cu") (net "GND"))
 (segment (start 186.74 90.885786) (end 186.74 92.72) (width 0.2) (layer "B.Cu") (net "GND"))
 (segment (start 179.36 118.6) (end 179.36 100.1) (width 0.2) (layer "B.Cu") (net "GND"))
 (segment (start 164.76 92.2) (end 168.26 88.7) (width 0.2) (layer "B.Cu") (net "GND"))
 (segment (start 180.56 90.2) (end 186.054214 90.2) (width 0.2) (layer "B.Cu") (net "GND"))
 (segment (start 186.054214 90.2) (end 186.74 90.885786) (width 0.2) (layer "B.Cu") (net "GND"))
 (segment (start 183.16 88.8) (end 185.74 86.22) (width 0.2) (layer "F.Cu") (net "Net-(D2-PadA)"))
 (segment (start 181.7 88.8) (end 183.16 88.8) (width 0.2) (layer "F.Cu") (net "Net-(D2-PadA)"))
 (segment (start 173 92.925786) (end 173 107.16) (width 0.2) (layer "B.Cu") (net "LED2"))
 (segment (start 185.74 91.3) (end 185.04 90.6) (width 0.2) (layer "B.Cu") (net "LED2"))
 (segment (start 175.325786 90.6) (end 173 92.925786) (width 0.2) (layer "B.Cu") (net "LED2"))
 (segment (start 185.04 90.6) (end 175.325786 90.6) (width 0.2) (layer "B.Cu") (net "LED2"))
 (segment (start 183.86 100.1) (end 186.34 97.62) (width 0.2) (layer "F.Cu") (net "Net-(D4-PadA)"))
 (segment (start 181.9 100.1) (end 183.86 100.1) (width 0.2) (layer "F.Cu") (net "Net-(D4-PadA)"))
 (segment (start 186.34 102.7) (end 187.04 103.4) (width 0.2) (layer "F.Cu") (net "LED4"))
 (segment (start 187.04 103.4) (end 187.04 107.321895) (width 0.2) (layer "F.Cu") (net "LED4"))
 (segment (start 187.04 107.321895) (end 186.139895 108.222) (width 0.2) (layer "F.Cu") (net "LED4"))
 (segment (start 186.139895 108.222) (end 184.638 108.222) (width 0.2) (layer "F.Cu") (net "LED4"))
 (segment (start 184.638 108.222) (end 170.46 122.4) (width 0.2) (layer "F.Cu") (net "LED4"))
 (segment (start 176.6 93.22) (end 176.6 106.1) (width 0.2) (layer "B.Cu") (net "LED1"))
 (segment (start 176.6 106.1) (end 175.54 107.16) (width 0.2) (layer "B.Cu") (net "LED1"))
 (segment (start 175.36 91.98) (end 176.6 93.22) (width 0.2) (layer "B.Cu") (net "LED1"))
 (segment (start 170.8 88.7) (end 173.56 88.7) (width 0.2) (layer "F.Cu") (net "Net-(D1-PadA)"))
 (segment (start 173.56 88.7) (end 175.36 86.9) (width 0.2) (layer "F.Cu") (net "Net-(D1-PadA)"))
 (segment (start 141.15 88.26) (end 162.133348 88.26) (width 0.2) (layer "F.Cu") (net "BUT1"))
 (segment (start 180.6 100.98237) (end 185.7 106.08237) (width 0.2) (layer "F.Cu") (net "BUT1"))
 (segment (start 185.7 106.08237) (end 185.7 107.16) (width 0.2) (layer "F.Cu") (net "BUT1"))
 (segment (start 180.6 98.925) (end 180.6 100.98237) (width 0.2) (layer "F.Cu") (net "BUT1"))
 (segment (start 162.133348 88.26) (end 170.693348 96.82) (width 0.2) (layer "F.Cu") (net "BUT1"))
 (segment (start 178.495 96.82) (end 180.6 98.925) (width 0.2) (layer "F.Cu") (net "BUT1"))
 (segment (start 170.693348 96.82) (end 178.495 96.82) (width 0.2) (layer "F.Cu") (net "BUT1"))
 (segment (start 139.75 89.66) (end 141.15 88.26) (width 0.2) (layer "F.Cu") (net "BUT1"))
 (segment (start 158.79 89.66) (end 162.967663 89.66) (width 0.2) (layer "F.Cu") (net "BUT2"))
 (segment (start 181.88663 104.809) (end 183.16 106.08237) (width 0.2) (layer "F.Cu") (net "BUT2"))
 (segment (start 183.16 106.08237) (end 183.16 107.16) (width 0.2) (layer "F.Cu") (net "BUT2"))
 (segment (start 174.701337 104.809) (end 181.88663 104.809) (width 0.2) (layer "F.Cu") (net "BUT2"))
 (segment (start 162.967663 89.66) (end 169.9925 96.684837) (width 0.2) (layer "F.Cu") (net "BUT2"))
 (segment (start 169.9925 100.100163) (end 174.701337 104.809) (width 0.2) (layer "F.Cu") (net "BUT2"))
 (segment (start 169.9925 96.684837) (end 169.9925 100.100163) (width 0.2) (layer "F.Cu") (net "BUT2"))
 (segment (start 156.880101 109.42) (end 158.280101 110.82) (width 0.2) (layer "F.Cu") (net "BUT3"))
 (segment (start 158.280101 110.82) (end 176.96 110.82) (width 0.2) (layer "F.Cu") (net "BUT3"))
 (segment (start 176.96 110.82) (end 180.62 107.16) (width 0.2) (layer "F.Cu") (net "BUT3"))
 (segment (start 139.76 109.42) (end 156.880101 109.42) (width 0.2) (layer "F.Cu") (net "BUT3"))
 (segment (start 158.86 109.42) (end 175.82 109.42) (width 0.2) (layer "F.Cu") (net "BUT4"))
 (segment (start 175.82 109.42) (end 178.08 107.16) (width 0.2) (layer "F.Cu") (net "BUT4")))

